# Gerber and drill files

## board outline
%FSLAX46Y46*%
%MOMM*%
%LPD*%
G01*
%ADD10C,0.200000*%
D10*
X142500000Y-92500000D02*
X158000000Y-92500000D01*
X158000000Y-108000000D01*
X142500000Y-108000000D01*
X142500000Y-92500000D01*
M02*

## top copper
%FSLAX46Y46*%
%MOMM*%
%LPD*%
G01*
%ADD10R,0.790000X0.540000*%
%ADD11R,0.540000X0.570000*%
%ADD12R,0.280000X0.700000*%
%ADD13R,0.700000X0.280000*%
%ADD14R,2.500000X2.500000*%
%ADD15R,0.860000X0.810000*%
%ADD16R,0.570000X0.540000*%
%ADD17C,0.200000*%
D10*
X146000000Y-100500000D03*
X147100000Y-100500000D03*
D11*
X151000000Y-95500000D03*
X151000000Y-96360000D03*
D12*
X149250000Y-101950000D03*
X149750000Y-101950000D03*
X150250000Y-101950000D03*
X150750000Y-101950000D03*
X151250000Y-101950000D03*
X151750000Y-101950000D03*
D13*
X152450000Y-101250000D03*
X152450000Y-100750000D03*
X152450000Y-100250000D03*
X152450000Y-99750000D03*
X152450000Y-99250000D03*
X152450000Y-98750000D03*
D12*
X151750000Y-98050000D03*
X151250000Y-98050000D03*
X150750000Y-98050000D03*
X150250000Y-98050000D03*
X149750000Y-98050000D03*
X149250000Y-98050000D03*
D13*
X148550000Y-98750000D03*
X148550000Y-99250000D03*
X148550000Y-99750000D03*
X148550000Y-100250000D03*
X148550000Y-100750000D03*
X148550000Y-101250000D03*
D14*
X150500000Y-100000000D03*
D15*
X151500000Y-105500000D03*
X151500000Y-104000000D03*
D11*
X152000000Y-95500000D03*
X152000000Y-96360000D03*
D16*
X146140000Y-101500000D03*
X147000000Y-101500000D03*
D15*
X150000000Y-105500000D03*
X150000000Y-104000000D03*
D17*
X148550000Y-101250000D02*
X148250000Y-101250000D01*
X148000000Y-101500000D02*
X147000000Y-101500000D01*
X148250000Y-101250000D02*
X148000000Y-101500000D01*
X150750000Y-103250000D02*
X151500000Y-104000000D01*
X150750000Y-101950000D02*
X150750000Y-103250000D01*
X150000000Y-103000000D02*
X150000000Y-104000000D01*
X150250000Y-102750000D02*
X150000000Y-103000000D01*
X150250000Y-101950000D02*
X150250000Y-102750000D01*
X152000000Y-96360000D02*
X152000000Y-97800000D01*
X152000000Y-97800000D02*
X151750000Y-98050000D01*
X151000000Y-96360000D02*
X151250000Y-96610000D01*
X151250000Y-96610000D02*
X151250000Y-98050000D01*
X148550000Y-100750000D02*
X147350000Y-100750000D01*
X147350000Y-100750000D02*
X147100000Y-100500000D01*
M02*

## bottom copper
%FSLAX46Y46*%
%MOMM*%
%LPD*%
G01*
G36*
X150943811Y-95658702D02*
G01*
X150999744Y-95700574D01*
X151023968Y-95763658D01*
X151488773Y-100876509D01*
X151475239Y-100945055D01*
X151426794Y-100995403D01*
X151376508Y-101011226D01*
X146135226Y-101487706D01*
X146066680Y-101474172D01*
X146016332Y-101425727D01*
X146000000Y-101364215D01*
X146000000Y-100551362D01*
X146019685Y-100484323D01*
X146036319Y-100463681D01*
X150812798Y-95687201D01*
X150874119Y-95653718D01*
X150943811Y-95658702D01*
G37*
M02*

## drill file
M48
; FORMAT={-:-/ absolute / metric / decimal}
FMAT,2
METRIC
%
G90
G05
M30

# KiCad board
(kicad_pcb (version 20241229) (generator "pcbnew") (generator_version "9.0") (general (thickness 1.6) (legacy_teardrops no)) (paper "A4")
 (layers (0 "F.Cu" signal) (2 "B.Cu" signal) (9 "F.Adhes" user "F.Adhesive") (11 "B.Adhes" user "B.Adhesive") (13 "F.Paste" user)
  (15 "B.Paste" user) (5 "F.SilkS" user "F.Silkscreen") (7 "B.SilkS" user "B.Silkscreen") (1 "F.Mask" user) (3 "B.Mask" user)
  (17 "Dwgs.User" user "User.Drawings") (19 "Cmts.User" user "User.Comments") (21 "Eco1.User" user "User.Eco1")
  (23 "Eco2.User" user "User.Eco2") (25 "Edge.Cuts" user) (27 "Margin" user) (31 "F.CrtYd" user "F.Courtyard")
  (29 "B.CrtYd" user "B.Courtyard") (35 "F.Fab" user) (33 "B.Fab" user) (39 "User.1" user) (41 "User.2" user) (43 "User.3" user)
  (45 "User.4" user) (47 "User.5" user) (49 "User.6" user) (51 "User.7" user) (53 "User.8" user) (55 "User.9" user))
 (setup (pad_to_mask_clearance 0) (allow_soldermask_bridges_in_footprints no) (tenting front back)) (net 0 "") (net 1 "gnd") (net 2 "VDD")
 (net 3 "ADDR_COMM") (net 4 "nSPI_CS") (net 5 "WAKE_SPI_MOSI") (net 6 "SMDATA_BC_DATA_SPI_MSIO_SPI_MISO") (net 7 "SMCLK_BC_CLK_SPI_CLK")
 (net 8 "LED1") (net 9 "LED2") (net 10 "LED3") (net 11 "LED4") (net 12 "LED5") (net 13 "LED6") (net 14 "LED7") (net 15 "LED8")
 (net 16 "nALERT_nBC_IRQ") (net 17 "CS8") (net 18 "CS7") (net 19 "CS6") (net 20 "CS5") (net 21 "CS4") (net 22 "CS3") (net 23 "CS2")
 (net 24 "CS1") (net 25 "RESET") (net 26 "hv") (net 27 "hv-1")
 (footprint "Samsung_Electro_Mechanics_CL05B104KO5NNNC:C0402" (layer "F.Cu") (at 146.55 100.5 180)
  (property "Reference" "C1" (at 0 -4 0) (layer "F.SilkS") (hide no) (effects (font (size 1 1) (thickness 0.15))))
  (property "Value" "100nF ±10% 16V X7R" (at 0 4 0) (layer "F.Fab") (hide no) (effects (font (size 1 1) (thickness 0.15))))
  (pad "2" smd rect (at 0.55 0 180) (size 0.79 0.54) (layers "F.Cu" "F.Paste" "F.Mask") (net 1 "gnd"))
  (pad "1" smd rect (at -0.55 0 180) (size 0.79 0.54) (layers "F.Cu" "F.Paste" "F.Mask") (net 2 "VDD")))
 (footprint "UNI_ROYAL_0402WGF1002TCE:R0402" (layer "F.Cu") (at 151 95.93 90)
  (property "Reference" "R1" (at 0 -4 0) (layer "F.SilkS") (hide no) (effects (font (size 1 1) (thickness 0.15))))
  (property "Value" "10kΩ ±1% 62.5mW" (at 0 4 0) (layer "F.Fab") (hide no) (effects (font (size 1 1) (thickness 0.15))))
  (pad "2" smd rect (at 0.43 0 90) (size 0.57 0.54) (layers "F.Cu" "F.Paste" "F.Mask") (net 1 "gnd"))
  (pad "1" smd rect (at -0.43 0 90) (size 0.57 0.54) (layers "F.Cu" "F.Paste" "F.Mask") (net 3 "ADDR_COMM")))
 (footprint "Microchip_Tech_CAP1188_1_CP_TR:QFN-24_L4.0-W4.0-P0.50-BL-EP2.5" (layer "F.Cu") (at 150.5 100 0)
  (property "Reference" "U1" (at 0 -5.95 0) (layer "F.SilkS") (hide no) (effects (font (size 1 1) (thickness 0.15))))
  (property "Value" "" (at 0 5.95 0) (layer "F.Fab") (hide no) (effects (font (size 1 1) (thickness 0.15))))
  (pad "1" smd rect (at -1.25 1.95 180) (size 0.28 0.7) (layers "F.Cu" "F.Mask" "F.Paste") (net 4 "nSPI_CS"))
  (pad "2" smd rect (at -0.75 1.95 180) (size 0.28 0.7) (layers "F.Cu" "F.Mask" "F.Paste") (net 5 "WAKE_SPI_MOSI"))
  (pad "3" smd rect (at -0.25 1.95 180) (size 0.28 0.7) (layers "F.Cu" "F.Mask" "F.Paste") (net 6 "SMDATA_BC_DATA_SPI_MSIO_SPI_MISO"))
  (pad "4" smd rect (at 0.25 1.95 180) (size 0.28 0.7) (layers "F.Cu" "F.Mask" "F.Paste") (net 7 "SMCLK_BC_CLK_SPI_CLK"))
  (pad "5" smd rect (at 0.75 1.95 180) (size 0.28 0.7) (layers "F.Cu" "F.Mask" "F.Paste") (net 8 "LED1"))
  (pad "6" smd rect (at 1.25 1.95 180) (size 0.28 0.7) (layers "F.Cu" "F.Mask" "F.Paste") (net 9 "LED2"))
  (pad "7" smd rect (at 1.95 1.25 270) (size 0.28 0.7) (layers "F.Cu" "F.Mask" "F.Paste") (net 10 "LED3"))
  (pad "8" smd rect (at 1.95 0.75 270) (size 0.28 0.7) (layers "F.Cu" "F.Mask" "F.Paste") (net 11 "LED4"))
  (pad "9" smd rect (at 1.95 0.25 270) (size 0.28 0.7) (layers "F.Cu" "F.Mask" "F.Paste") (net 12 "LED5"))
  (pad "10" smd rect (at 1.95 -0.25 270) (size 0.28 0.7) (layers "F.Cu" "F.Mask" "F.Paste") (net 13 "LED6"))
  (pad "11" smd rect (at 1.95 -0.75 270) (size 0.28 0.7) (layers "F.Cu" "F.Mask" "F.Paste") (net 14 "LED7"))
  (pad "12" smd rect (at 1.95 -1.25 270) (size 0.28 0.7) (layers "F.Cu" "F.Mask" "F.Paste") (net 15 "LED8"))
  (pad "13" smd rect (at 1.25 -1.95 0) (size 0.28 0.7) (layers "F.Cu" "F.Mask" "F.Paste") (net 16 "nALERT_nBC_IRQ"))
  (pad "14" smd rect (at 0.75 -1.95 0) (size 0.28 0.7) (layers "F.Cu" "F.Mask" "F.Paste") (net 3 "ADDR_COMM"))
  (pad "15" smd rect (at 0.25 -1.95 0) (size 0.28 0.7) (layers "F.Cu" "F.Mask" "F.Paste") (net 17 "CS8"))
  (pad "16" smd rect (at -0.25 -1.95 0) (size 0.28 0.7) (layers "F.Cu" "F.Mask" "F.Paste") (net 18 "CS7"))
  (pad "17" smd rect (at -0.75 -1.95 0) (size 0.28 0.7) (layers "F.Cu" "F.Mask" "F.Paste") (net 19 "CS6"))
  (pad "18" smd rect (at -1.25 -1.95 0) (size 0.28 0.7) (layers "F.Cu" "F.Mask" "F.Paste") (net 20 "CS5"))
  (pad "19" smd rect (at -1.95 -1.25 90) (size 0.28 0.7) (layers "F.Cu" "F.Mask" "F.Paste") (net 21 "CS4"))
  (pad "20" smd rect (at -1.95 -0.75 90) (size 0.28 0.7) (layers "F.Cu" "F.Mask" "F.Paste") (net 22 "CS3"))
  (pad "21" smd rect (at -1.95 -0.25 90) (size 0.28 0.7) (layers "F.Cu" "F.Mask" "F.Paste") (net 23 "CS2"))
  (pad "22" smd rect (at -1.95 0.25 90) (size 0.28 0.7) (layers "F.Cu" "F.Mask" "F.Paste") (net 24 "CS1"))
  (pad "23" smd rect (at -1.95 0.75 90) (size 0.28 0.7) (layers "F.Cu" "F.Mask" "F.Paste") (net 2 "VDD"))
  (pad "24" smd rect (at -1.95 1.25 90) (size 0.28 0.7) (layers "F.Cu" "F.Mask" "F.Paste") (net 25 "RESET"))
  (pad "25" smd rect (at 0 0 90) (size 2.5 2.5) (layers "F.Cu" "F.Mask" "F.Paste") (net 1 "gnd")))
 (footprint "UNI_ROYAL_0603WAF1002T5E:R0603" (layer "F.Cu") (at 151.5 104.75 -90)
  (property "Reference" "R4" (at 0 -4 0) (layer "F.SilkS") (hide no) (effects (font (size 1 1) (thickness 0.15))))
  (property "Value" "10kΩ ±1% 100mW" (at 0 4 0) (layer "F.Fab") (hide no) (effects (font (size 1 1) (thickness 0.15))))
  (pad "2" smd rect (at 0.75 0 -90) (size 0.81 0.86) (layers "F.Cu" "F.Paste" "F.Mask") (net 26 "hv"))
  (pad "1" smd rect (at -0.75 0 -90) (size 0.81 0.86) (layers "F.Cu" "F.Paste" "F.Mask") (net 7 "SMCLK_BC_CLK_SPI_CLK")))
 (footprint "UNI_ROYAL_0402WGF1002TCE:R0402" (layer "F.Cu") (at 152 95.93 90)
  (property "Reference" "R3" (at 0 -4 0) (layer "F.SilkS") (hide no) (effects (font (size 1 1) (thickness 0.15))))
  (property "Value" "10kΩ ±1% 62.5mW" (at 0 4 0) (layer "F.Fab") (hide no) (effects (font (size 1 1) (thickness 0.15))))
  (pad "2" smd rect (at 0.43 0 90) (size 0.57 0.54) (layers "F.Cu" "F.Paste" "F.Mask") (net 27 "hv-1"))
  (pad "1" smd rect (at -0.43 0 90) (size 0.57 0.54) (layers "F.Cu" "F.Paste" "F.Mask") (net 16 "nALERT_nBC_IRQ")))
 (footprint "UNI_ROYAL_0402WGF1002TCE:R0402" (layer "F.Cu") (at 146.57 101.5 180)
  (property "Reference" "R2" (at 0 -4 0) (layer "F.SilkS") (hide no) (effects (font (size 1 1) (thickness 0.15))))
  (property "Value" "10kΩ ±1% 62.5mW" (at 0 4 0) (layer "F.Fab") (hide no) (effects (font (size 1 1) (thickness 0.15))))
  (pad "2" smd rect (at 0.43 0 180) (size 0.57 0.54) (layers "F.Cu" "F.Paste" "F.Mask") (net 1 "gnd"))
  (pad "1" smd rect (at -0.43 0 180) (size 0.57 0.54) (layers "F.Cu" "F.Paste" "F.Mask") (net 25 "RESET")))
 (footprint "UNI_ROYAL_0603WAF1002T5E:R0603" (layer "F.Cu") (at 150 104.75 -90)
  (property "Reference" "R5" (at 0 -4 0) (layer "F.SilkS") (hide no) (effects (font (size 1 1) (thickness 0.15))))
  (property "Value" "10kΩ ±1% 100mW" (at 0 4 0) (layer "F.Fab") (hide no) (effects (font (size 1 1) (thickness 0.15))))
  (pad "2" smd rect (at 0.75 0 -90) (size 0.81 0.86) (layers "F.Cu" "F.Paste" "F.Mask") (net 26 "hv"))
  (pad "1" smd rect (at -0.75 0 -90) (size 0.81 0.86) (layers "F.Cu" "F.Paste" "F.Mask") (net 6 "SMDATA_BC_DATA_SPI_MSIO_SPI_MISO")))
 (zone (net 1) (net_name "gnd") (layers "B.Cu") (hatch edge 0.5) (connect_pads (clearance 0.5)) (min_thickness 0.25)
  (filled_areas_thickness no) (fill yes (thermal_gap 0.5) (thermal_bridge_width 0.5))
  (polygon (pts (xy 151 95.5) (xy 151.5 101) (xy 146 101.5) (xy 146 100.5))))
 (segment (start 148.55 101.25) (end 148.25 101.25) (width 0.2) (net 25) (layer "F.Cu"))
 (segment (start 148 101.5) (end 147 101.5) (width 0.2) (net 25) (layer "F.Cu"))
 (segment (start 148.25 101.25) (end 148 101.5) (width 0.2) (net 25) (layer "F.Cu"))
 (segment (start 150.75 103.25) (end 151.5 104) (width 0.2) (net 7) (layer "F.Cu"))
 (segment (start 150.75 101.95) (end 150.75 103.25) (width 0.2) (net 7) (layer "F.Cu"))
 (segment (start 150 103) (end 150 104) (width 0.2) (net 6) (layer "F.Cu"))
 (segment (start 150.25 102.75) (end 150 103) (width 0.2) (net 6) (layer "F.Cu"))
 (segment (start 150.25 101.95) (end 150.25 102.75) (width 0.2) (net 6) (layer "F.Cu"))
 (segment (start 152 96.36) (end 152 97.8) (width 0.2) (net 16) (layer "F.Cu"))
 (segment (start 152 97.8) (end 151.75 98.05) (width 0.2) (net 16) (layer "F.Cu"))
 (segment (start 151 96.36) (end 151.25 96.61) (width 0.2) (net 3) (layer "F.Cu"))
 (segment (start 151.25 96.61) (end 151.25 98.05) (width 0.2) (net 3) (layer "F.Cu"))
 (segment (start 148.55 100.75) (end 147.35 100.75) (width 0.2) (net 2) (layer "F.Cu"))
 (segment (start 147.35 100.75) (end 147.1 100.5) (width 0.2) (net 2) (layer "F.Cu"))
 (gr_rect (start 142.5 92.5) (end 158 108) (stroke (width 0.2) (type solid)) (fill no) (layer "Edge.Cuts")))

